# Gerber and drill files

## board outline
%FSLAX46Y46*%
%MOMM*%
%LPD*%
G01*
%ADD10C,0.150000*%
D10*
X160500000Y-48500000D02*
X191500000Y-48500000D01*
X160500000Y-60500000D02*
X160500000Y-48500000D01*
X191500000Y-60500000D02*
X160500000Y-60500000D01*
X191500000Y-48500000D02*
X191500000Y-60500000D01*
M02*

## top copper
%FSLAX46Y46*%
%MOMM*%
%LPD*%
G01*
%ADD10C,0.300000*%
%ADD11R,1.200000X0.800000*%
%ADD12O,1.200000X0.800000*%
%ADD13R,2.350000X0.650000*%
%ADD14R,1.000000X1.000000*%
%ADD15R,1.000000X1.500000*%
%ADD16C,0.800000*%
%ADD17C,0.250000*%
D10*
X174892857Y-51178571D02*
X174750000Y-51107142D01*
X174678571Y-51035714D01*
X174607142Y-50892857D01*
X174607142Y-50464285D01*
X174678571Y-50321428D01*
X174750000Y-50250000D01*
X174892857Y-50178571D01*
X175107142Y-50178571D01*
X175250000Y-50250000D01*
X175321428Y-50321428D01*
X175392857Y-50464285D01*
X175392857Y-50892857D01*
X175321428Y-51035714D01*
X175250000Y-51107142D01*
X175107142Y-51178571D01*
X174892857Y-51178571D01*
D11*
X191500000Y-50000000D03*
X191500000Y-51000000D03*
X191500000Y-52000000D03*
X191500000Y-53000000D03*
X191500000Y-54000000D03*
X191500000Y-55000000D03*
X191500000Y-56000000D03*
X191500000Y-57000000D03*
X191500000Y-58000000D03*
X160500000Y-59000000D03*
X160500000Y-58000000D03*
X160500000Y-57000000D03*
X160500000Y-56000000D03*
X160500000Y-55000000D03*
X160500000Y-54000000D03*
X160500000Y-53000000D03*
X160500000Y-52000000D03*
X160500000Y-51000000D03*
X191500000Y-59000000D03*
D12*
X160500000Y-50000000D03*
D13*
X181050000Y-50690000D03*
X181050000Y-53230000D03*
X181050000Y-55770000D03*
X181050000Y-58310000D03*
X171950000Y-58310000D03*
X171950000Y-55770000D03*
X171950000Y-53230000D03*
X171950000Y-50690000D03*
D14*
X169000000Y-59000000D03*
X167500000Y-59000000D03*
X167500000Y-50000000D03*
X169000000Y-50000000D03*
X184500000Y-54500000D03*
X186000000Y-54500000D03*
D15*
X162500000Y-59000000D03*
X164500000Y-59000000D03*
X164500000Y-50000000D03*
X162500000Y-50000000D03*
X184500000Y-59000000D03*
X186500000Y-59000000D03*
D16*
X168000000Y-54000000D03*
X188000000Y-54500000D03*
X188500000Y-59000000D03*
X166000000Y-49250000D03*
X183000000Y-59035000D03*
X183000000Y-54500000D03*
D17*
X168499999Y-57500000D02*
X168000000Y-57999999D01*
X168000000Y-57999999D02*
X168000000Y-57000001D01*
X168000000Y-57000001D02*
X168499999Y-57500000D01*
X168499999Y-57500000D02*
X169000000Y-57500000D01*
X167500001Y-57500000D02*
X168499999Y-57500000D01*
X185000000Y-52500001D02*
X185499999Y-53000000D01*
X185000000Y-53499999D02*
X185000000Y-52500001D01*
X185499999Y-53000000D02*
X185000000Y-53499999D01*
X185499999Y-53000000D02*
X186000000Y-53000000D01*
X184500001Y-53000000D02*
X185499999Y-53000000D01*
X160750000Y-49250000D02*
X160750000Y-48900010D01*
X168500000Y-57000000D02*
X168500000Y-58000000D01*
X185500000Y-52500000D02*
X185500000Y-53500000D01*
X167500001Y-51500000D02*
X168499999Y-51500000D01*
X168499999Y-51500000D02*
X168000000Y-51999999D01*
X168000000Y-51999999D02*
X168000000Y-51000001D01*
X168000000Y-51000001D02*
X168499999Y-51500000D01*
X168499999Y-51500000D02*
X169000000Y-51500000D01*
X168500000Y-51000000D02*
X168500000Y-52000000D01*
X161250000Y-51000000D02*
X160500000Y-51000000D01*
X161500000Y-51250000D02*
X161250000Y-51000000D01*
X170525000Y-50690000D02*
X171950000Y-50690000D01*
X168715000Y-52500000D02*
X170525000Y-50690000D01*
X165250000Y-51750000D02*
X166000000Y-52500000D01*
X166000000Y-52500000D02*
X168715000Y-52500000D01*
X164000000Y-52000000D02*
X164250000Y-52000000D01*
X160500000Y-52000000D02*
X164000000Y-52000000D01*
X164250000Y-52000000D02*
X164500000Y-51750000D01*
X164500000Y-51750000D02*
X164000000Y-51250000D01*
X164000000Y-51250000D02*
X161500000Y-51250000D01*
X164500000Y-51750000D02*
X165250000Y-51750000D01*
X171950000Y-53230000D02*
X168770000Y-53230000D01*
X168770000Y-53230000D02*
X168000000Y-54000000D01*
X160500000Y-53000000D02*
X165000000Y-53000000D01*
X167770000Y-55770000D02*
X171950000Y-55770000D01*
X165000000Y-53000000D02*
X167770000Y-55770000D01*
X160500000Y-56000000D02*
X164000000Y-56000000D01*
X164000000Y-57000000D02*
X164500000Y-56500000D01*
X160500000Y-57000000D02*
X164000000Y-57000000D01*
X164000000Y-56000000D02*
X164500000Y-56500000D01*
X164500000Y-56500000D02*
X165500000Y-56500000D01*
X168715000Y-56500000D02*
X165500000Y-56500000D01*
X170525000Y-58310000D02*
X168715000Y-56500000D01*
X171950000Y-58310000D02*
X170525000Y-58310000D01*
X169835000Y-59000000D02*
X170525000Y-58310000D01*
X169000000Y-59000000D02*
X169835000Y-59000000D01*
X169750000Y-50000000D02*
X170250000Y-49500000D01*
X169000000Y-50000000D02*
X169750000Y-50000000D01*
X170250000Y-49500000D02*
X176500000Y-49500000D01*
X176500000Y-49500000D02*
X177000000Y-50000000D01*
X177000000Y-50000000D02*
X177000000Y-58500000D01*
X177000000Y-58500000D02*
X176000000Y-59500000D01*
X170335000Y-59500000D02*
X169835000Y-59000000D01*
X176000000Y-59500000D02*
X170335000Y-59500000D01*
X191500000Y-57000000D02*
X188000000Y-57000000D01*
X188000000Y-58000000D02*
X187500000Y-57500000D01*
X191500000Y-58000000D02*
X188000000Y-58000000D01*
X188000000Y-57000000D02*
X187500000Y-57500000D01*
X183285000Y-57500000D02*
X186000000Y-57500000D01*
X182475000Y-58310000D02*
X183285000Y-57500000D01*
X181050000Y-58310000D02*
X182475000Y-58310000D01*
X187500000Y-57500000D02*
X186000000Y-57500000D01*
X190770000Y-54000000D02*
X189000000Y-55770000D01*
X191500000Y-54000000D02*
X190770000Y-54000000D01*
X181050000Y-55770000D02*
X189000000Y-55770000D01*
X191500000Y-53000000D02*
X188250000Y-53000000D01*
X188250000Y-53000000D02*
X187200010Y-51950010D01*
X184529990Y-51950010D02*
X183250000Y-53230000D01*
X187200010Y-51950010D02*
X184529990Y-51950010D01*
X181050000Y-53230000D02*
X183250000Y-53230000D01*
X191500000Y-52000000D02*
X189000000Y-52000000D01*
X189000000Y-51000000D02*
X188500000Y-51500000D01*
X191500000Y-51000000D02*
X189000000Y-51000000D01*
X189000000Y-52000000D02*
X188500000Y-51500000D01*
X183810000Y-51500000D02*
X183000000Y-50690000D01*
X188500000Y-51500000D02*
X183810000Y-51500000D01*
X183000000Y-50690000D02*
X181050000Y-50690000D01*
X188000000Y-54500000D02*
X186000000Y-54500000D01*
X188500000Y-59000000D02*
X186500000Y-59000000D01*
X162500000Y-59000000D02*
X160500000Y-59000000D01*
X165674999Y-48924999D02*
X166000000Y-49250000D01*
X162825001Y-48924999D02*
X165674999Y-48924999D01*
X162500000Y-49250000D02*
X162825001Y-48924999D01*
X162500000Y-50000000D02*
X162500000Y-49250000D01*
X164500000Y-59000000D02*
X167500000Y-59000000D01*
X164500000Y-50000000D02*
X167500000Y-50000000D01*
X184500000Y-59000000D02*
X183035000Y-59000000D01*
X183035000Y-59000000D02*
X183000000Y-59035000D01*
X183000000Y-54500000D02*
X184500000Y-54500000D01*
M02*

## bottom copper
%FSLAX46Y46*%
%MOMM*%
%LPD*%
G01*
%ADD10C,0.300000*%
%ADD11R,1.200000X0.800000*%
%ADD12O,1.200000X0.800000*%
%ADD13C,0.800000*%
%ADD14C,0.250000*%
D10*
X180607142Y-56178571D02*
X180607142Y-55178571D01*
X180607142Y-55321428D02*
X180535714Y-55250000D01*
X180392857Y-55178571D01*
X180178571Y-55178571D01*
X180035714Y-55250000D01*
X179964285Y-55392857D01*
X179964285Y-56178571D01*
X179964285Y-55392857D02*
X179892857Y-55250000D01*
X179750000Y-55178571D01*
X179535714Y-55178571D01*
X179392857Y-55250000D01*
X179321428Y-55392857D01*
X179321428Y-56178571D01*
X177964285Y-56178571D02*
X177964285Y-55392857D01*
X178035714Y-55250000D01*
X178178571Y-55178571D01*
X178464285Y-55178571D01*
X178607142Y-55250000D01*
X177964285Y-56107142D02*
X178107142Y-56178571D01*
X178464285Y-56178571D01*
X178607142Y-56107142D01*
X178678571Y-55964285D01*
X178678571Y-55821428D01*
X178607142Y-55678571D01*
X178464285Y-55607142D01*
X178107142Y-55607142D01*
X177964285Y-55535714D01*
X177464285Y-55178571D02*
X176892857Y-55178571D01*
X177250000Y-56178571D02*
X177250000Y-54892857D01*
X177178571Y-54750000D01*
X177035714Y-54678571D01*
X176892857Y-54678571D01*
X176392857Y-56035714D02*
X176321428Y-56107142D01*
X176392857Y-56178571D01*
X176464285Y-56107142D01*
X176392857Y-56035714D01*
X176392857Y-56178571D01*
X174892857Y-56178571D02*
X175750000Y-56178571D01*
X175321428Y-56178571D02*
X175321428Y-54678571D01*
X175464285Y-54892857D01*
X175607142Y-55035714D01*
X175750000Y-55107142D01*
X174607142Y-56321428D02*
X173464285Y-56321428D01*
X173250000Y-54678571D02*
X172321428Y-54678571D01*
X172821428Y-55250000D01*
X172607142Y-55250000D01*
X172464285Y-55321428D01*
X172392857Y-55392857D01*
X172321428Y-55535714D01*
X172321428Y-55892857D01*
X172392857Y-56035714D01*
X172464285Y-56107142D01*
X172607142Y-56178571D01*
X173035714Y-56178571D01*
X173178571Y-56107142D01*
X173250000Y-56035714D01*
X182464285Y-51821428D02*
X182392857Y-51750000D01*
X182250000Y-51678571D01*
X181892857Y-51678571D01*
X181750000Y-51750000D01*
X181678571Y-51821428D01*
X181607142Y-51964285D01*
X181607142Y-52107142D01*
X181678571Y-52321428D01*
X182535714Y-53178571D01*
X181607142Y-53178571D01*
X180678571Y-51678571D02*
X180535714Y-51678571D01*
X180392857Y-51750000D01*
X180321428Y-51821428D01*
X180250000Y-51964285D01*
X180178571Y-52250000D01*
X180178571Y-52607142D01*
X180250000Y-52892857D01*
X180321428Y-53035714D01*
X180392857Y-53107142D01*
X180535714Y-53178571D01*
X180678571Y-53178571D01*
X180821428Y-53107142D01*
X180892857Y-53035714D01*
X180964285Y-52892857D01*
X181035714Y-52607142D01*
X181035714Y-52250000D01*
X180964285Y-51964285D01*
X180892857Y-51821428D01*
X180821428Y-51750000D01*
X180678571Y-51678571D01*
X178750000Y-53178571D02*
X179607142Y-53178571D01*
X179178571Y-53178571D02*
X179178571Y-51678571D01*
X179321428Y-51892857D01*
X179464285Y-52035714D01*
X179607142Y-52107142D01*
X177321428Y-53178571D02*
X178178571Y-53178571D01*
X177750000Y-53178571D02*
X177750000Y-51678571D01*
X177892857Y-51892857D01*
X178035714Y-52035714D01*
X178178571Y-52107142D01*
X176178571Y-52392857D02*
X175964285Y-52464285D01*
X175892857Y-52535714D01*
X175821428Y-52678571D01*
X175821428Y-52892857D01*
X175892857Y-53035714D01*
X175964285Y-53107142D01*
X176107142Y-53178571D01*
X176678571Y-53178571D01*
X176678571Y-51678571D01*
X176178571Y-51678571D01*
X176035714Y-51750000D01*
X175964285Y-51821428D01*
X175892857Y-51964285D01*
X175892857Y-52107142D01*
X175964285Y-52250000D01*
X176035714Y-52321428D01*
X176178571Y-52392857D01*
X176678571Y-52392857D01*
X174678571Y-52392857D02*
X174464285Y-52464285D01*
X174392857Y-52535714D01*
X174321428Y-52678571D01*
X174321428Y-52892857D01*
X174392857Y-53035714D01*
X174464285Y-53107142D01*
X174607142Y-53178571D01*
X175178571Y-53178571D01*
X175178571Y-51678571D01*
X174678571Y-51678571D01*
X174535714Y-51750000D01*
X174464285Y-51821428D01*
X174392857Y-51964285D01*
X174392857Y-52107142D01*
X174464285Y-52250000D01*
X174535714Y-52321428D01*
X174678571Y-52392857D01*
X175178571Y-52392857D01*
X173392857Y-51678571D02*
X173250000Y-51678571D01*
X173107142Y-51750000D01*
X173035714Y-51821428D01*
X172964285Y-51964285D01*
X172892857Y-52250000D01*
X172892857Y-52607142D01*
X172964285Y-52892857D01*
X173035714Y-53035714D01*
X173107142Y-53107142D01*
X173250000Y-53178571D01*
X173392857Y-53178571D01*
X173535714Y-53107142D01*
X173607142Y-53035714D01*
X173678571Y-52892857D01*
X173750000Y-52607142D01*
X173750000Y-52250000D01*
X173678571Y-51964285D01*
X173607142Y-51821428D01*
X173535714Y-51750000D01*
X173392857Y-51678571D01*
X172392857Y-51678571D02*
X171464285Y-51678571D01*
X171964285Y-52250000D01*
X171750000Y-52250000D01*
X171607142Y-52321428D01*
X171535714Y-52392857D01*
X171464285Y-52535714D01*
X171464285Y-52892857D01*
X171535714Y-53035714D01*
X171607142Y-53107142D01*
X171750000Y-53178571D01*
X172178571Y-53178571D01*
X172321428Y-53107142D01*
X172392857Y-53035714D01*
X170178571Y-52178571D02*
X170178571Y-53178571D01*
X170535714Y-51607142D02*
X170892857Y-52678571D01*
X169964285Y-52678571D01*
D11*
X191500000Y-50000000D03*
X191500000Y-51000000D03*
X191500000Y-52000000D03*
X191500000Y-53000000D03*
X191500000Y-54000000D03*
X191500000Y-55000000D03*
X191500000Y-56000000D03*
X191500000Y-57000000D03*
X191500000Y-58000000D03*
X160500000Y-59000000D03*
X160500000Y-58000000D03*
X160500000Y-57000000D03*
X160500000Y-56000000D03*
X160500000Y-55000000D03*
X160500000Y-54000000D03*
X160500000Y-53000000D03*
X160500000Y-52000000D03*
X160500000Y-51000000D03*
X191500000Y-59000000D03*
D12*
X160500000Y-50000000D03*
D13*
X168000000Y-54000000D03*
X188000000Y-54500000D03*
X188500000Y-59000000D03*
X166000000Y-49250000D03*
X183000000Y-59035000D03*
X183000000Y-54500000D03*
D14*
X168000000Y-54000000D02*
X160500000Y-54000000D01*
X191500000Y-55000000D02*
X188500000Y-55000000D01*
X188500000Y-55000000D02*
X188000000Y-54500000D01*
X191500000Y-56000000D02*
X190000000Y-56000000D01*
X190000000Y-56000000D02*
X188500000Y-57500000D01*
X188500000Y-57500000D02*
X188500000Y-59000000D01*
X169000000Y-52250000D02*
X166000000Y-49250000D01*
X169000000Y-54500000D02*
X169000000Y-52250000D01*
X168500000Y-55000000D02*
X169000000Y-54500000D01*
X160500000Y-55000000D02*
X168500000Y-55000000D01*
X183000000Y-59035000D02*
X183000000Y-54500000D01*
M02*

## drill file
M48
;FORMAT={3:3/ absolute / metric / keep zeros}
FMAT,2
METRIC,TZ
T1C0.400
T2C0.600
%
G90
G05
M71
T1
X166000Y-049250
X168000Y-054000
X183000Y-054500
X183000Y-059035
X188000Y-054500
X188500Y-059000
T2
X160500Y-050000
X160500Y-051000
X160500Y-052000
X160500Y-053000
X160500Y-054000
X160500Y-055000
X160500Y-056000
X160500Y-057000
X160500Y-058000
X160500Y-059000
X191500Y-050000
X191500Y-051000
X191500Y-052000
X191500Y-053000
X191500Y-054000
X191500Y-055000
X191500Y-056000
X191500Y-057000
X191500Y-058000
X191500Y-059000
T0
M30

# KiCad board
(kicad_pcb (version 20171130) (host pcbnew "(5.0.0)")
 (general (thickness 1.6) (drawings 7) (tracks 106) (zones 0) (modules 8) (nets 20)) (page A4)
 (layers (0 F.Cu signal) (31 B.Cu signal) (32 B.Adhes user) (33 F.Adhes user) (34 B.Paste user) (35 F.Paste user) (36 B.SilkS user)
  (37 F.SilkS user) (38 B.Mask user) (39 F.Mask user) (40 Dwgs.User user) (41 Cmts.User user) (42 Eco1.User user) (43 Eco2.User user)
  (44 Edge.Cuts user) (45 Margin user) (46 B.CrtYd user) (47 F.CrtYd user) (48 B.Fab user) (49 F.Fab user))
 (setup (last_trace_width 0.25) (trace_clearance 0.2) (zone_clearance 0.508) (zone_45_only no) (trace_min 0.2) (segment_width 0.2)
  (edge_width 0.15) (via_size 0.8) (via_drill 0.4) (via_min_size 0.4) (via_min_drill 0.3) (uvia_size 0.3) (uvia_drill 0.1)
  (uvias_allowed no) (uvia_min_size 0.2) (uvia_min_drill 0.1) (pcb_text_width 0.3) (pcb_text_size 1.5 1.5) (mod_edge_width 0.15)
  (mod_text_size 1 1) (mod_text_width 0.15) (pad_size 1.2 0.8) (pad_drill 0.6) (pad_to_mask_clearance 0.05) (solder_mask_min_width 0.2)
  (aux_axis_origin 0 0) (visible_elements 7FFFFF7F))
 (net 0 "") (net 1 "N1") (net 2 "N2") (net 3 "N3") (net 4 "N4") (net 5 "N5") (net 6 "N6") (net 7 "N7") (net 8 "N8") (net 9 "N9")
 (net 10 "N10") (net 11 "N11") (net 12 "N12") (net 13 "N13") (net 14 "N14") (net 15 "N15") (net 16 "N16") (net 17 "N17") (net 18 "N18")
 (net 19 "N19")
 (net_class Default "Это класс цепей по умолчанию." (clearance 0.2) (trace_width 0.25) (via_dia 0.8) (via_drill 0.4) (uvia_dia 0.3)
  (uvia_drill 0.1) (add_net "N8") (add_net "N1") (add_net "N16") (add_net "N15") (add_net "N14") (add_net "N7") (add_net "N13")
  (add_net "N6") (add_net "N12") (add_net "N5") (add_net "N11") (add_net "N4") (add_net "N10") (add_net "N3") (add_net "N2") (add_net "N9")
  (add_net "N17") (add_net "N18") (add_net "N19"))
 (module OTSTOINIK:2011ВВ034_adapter (layer F.Cu) (at 176 54.5)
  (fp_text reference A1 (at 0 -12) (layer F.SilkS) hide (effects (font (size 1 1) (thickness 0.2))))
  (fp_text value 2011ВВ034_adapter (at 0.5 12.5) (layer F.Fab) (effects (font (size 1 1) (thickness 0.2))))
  (pad 10B thru_hole rect (at 15.5 -4.5) (size 1.2 0.8) (drill 0.6) (layers *.Cu *.Mask) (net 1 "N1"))
  (pad 9B thru_hole rect (at 15.5 -3.5) (size 1.2 0.8) (drill 0.6) (layers *.Cu *.Mask) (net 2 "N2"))
  (pad 8B thru_hole rect (at 15.5 -2.5) (size 1.2 0.8) (drill 0.6) (layers *.Cu *.Mask) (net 2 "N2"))
  (pad 7B thru_hole rect (at 15.5 -1.5) (size 1.2 0.8) (drill 0.6) (layers *.Cu *.Mask) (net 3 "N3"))
  (pad 6B thru_hole rect (at 15.5 -0.5) (size 1.2 0.8) (drill 0.6) (layers *.Cu *.Mask) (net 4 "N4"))
  (pad 5B thru_hole rect (at 15.5 0.5) (size 1.2 0.8) (drill 0.6) (layers *.Cu *.Mask) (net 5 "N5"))
  (pad 4B thru_hole rect (at 15.5 1.5) (size 1.2 0.8) (drill 0.6) (layers *.Cu *.Mask) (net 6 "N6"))
  (pad 3B thru_hole rect (at 15.5 2.5) (size 1.2 0.8) (drill 0.6) (layers *.Cu *.Mask) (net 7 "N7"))
  (pad 2B thru_hole rect (at 15.5 3.5) (size 1.2 0.8) (drill 0.6) (layers *.Cu *.Mask) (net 7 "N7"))
  (pad 10A thru_hole rect (at -15.5 4.5) (size 1.2 0.8) (drill 0.6) (layers *.Cu *.Mask) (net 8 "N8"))
  (pad 9A thru_hole rect (at -15.5 3.5) (size 1.2 0.8) (drill 0.6) (layers *.Cu *.Mask) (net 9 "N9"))
  (pad 8A thru_hole rect (at -15.5 2.5) (size 1.2 0.8) (drill 0.6) (layers *.Cu *.Mask) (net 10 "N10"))
  (pad 7A thru_hole rect (at -15.5 1.5) (size 1.2 0.8) (drill 0.6) (layers *.Cu *.Mask) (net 10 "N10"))
  (pad 6A thru_hole rect (at -15.5 0.5) (size 1.2 0.8) (drill 0.6) (layers *.Cu *.Mask) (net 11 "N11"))
  (pad 5A thru_hole rect (at -15.5 -0.5) (size 1.2 0.8) (drill 0.6) (layers *.Cu *.Mask) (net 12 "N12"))
  (pad 4A thru_hole rect (at -15.5 -1.5) (size 1.2 0.8) (drill 0.6) (layers *.Cu *.Mask) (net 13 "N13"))
  (pad 3A thru_hole rect (at -15.5 -2.5) (size 1.2 0.8) (drill 0.6) (layers *.Cu *.Mask) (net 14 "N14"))
  (pad 2A thru_hole rect (at -15.5 -3.5) (size 1.2 0.8) (drill 0.6) (layers *.Cu *.Mask) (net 14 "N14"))
  (pad 1B thru_hole rect (at 15.5 4.5) (size 1.2 0.8) (drill 0.6) (layers *.Cu *.Mask) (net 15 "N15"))
  (pad 1A thru_hole oval (at -15.5 -4.5) (size 1.2 0.8) (drill 0.6) (layers *.Cu *.Mask) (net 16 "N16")))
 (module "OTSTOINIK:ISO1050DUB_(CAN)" (layer F.Cu) (at 176.5 54.5)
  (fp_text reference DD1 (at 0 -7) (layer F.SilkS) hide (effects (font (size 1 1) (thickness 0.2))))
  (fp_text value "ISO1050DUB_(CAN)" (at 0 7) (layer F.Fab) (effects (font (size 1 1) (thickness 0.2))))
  (pad 8 smd rect (at 4.55 -3.81) (size 2.35 0.65) (layers F.Cu F.Paste F.Mask) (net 2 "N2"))
  (pad 7 smd rect (at 4.55 -1.27) (size 2.35 0.65) (layers F.Cu F.Paste F.Mask) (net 3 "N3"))
  (pad 6 smd rect (at 4.55 1.27) (size 2.35 0.65) (layers F.Cu F.Paste F.Mask) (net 4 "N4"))
  (pad 5 smd rect (at 4.55 3.81) (size 2.35 0.65) (layers F.Cu F.Paste F.Mask) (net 7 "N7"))
  (pad 4 smd rect (at -4.55 3.81) (size 2.35 0.65) (layers F.Cu F.Paste F.Mask) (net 10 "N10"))
  (pad 3 smd rect (at -4.55 1.27) (size 2.35 0.65) (layers F.Cu F.Paste F.Mask) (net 13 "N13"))
  (pad 2 smd rect (at -4.55 -1.27) (size 2.35 0.65) (layers F.Cu F.Paste F.Mask) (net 12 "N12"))
  (pad 1 smd rect (at -4.55 -3.81) (size 2.35 0.65) (layers F.Cu F.Paste F.Mask) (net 14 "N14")))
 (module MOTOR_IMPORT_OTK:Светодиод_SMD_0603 (layer F.Cu) (at 167.5 59)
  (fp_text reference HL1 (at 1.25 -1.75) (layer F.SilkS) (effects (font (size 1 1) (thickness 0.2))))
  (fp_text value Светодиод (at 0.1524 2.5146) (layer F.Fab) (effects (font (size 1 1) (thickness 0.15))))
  (pad 2 smd rect (at 1.5 0) (size 1 1) (layers F.Cu F.Paste F.Mask) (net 10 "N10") (clearance 0.2))
  (pad 1 smd rect (at 0 0) (size 1 1) (layers F.Cu F.Paste F.Mask) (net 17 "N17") (clearance 0.2)))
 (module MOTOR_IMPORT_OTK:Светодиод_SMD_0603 (layer F.Cu) (at 167.5 50)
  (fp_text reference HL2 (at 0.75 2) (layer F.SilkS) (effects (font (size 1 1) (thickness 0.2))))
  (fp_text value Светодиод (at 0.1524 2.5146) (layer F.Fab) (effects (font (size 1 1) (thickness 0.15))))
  (pad 1 smd rect (at 0 0) (size 1 1) (layers F.Cu F.Paste F.Mask) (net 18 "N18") (clearance 0.2))
  (pad 2 smd rect (at 1.5 0) (size 1 1) (layers F.Cu F.Paste F.Mask) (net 10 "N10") (clearance 0.2)))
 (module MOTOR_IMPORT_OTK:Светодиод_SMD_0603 (layer F.Cu) (at 184.5 54.5)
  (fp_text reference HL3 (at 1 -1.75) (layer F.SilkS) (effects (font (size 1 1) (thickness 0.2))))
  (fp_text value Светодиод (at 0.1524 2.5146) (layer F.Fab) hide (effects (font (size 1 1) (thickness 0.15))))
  (pad 1 smd rect (at 0 0) (size 1 1) (layers F.Cu F.Paste F.Mask) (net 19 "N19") (clearance 0.2))
  (pad 2 smd rect (at 1.5 0) (size 1 1) (layers F.Cu F.Paste F.Mask) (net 5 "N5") (clearance 0.2)))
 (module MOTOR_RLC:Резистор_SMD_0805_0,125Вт (layer F.Cu) (at 164.5 59 180)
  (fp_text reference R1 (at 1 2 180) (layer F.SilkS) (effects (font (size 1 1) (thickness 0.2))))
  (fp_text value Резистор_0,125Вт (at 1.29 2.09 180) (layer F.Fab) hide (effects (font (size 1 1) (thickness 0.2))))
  (pad 2 smd rect (at 2 0 180) (size 1 1.5) (layers F.Cu F.Paste F.Mask) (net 8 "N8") (clearance 0.2))
  (pad 1 smd rect (at 0 0 180) (size 1 1.5) (layers F.Cu F.Paste F.Mask) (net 17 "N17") (clearance 0.2)))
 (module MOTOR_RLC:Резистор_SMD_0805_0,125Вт (layer F.Cu) (at 164.5 50 180)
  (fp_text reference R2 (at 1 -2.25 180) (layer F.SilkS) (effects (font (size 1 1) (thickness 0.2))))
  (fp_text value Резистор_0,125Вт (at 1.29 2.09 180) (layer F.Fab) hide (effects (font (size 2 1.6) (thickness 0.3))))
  (pad 1 smd rect (at 0 0 180) (size 1 1.5) (layers F.Cu F.Paste F.Mask) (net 18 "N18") (clearance 0.2))
  (pad 2 smd rect (at 2 0 180) (size 1 1.5) (layers F.Cu F.Paste F.Mask) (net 11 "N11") (clearance 0.2)))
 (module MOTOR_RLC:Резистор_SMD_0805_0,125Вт (layer F.Cu) (at 186.5 59 180)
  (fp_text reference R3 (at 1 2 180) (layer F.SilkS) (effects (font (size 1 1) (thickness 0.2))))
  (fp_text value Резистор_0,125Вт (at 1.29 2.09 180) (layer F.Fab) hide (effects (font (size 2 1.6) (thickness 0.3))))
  (pad 2 smd rect (at 2 0 180) (size 1 1.5) (layers F.Cu F.Paste F.Mask) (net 19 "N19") (clearance 0.2))
  (pad 1 smd rect (at 0 0 180) (size 1 1.5) (layers F.Cu F.Paste F.Mask) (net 6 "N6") (clearance 0.2)))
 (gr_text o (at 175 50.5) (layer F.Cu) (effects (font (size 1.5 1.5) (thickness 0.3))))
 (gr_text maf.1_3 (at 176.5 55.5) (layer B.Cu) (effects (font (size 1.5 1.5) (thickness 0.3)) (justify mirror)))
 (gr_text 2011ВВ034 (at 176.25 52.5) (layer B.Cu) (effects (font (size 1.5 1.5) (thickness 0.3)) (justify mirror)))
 (gr_line (start 160.5 48.5) (end 191.5 48.5) (layer Edge.Cuts) (width 0.15))
 (gr_line (start 160.5 60.5) (end 160.5 48.5) (layer Edge.Cuts) (width 0.15))
 (gr_line (start 191.5 60.5) (end 160.5 60.5) (layer Edge.Cuts) (width 0.15))
 (gr_line (start 191.5 48.5) (end 191.5 60.5) (layer Edge.Cuts) (width 0.15))
 (segment (start 168.499999 57.5) (end 168 57.999999) (width 0.25) (layer F.Cu) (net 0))
 (segment (start 168 57.999999) (end 168 57.000001) (width 0.25) (layer F.Cu) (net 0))
 (segment (start 168 57.000001) (end 168.499999 57.5) (width 0.25) (layer F.Cu) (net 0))
 (segment (start 168.499999 57.5) (end 169 57.5) (width 0.25) (layer F.Cu) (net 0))
 (segment (start 167.500001 57.5) (end 168.499999 57.5) (width 0.25) (layer F.Cu) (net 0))
 (segment (start 185 52.500001) (end 185.499999 53) (width 0.25) (layer F.Cu) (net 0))
 (segment (start 185 53.499999) (end 185 52.500001) (width 0.25) (layer F.Cu) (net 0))
 (segment (start 185.499999 53) (end 185 53.499999) (width 0.25) (layer F.Cu) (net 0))
 (segment (start 185.499999 53) (end 186 53) (width 0.25) (layer F.Cu) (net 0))
 (segment (start 184.500001 53) (end 185.499999 53) (width 0.25) (layer F.Cu) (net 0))
 (segment (start 160.75 49.25) (end 160.75 48.90001) (width 0.25) (layer F.Cu) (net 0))
 (segment (start 168.5 57) (end 168.5 58) (width 0.25) (layer F.Cu) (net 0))
 (segment (start 185.5 52.5) (end 185.5 53.5) (width 0.25) (layer F.Cu) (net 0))
 (segment (start 167.500001 51.5) (end 168.499999 51.5) (width 0.25) (layer F.Cu) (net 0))
 (segment (start 168.499999 51.5) (end 168 51.999999) (width 0.25) (layer F.Cu) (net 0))
 (segment (start 168 51.999999) (end 168 51.000001) (width 0.25) (layer F.Cu) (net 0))
 (segment (start 168 51.000001) (end 168.499999 51.5) (width 0.25) (layer F.Cu) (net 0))
 (segment (start 168.499999 51.5) (end 169 51.5) (width 0.25) (layer F.Cu) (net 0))
 (segment (start 168.5 51) (end 168.5 52) (width 0.25) (layer F.Cu) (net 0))
 (segment (start 161.25 51) (end 160.5 51) (width 0.25) (layer F.Cu) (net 14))
 (segment (start 161.5 51.25) (end 161.25 51) (width 0.25) (layer F.Cu) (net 14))
 (segment (start 170.525 50.69) (end 171.95 50.69) (width 0.25) (layer F.Cu) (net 14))
 (segment (start 168.715 52.5) (end 170.525 50.69) (width 0.25) (layer F.Cu) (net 14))
 (segment (start 165.25 51.75) (end 166 52.5) (width 0.25) (layer F.Cu) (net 14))
 (segment (start 166 52.5) (end 168.715 52.5) (width 0.25) (layer F.Cu) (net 14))
 (segment (start 164 52) (end 164.25 52) (width 0.25) (layer F.Cu) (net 14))
 (segment (start 160.5 52) (end 164 52) (width 0.25) (layer F.Cu) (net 14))
 (segment (start 164.25 52) (end 164.5 51.75) (width 0.25) (layer F.Cu) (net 14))
 (segment (start 164.5 51.75) (end 164 51.25) (width 0.25) (layer F.Cu) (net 14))
 (segment (start 164 51.25) (end 161.5 51.25) (width 0.25) (layer F.Cu) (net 14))
 (segment (start 164.5 51.75) (end 165.25 51.75) (width 0.25) (layer F.Cu) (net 14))
 (via (at 168 54) (size 0.8) (drill 0.4) (layers F.Cu B.Cu) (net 12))
 (segment (start 171.95 53.23) (end 168.77 53.23) (width 0.25) (layer F.Cu) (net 12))
 (segment (start 168.77 53.23) (end 168 54) (width 0.25) (layer F.Cu) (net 12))
 (segment (start 168 54) (end 160.5 54) (width 0.25) (layer B.Cu) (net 12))
 (segment (start 160.5 53) (end 165 53) (width 0.25) (layer F.Cu) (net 13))
 (segment (start 167.77 55.77) (end 171.95 55.77) (width 0.25) (layer F.Cu) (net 13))
 (segment (start 165 53) (end 167.77 55.77) (width 0.25) (layer F.Cu) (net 13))
 (segment (start 160.5 56) (end 164 56) (width 0.25) (layer F.Cu) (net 10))
 (segment (start 164 57) (end 164.5 56.5) (width 0.25) (layer F.Cu) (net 10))
 (segment (start 160.5 57) (end 164 57) (width 0.25) (layer F.Cu) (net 10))
 (segment (start 164 56) (end 164.5 56.5) (width 0.25) (layer F.Cu) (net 10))
 (segment (start 164.5 56.5) (end 165.5 56.5) (width 0.25) (layer F.Cu) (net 10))
 (segment (start 168.715 56.5) (end 165.5 56.5) (width 0.25) (layer F.Cu) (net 10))
 (segment (start 170.525 58.31) (end 168.715 56.5) (width 0.25) (layer F.Cu) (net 10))
 (segment (start 171.95 58.31) (end 170.525 58.31) (width 0.25) (layer F.Cu) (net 10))
 (segment (start 169.835 59) (end 170.525 58.31) (width 0.25) (layer F.Cu) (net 10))
 (segment (start 169 59) (end 169.835 59) (width 0.25) (layer F.Cu) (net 10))
 (segment (start 169.75 50) (end 170.25 49.5) (width 0.25) (layer F.Cu) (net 10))
 (segment (start 169 50) (end 169.75 50) (width 0.25) (layer F.Cu) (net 10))
 (segment (start 170.25 49.5) (end 176.5 49.5) (width 0.25) (layer F.Cu) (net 10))
 (segment (start 176.5 49.5) (end 177 50) (width 0.25) (layer F.Cu) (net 10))
 (segment (start 177 50) (end 177 58.5) (width 0.25) (layer F.Cu) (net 10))
 (segment (start 177 58.5) (end 176 59.5) (width 0.25) (layer F.Cu) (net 10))
 (segment (start 170.335 59.5) (end 169.835 59) (width 0.25) (layer F.Cu) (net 10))
 (segment (start 176 59.5) (end 170.335 59.5) (width 0.25) (layer F.Cu) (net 10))
 (segment (start 191.5 57) (end 188 57) (width 0.25) (layer F.Cu) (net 7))
 (segment (start 188 58) (end 187.5 57.5) (width 0.25) (layer F.Cu) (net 7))
 (segment (start 191.5 58) (end 188 58) (width 0.25) (layer F.Cu) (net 7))
 (segment (start 188 57) (end 187.5 57.5) (width 0.25) (layer F.Cu) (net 7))
 (segment (start 183.285 57.5) (end 186 57.5) (width 0.25) (layer F.Cu) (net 7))
 (segment (start 182.475 58.31) (end 183.285 57.5) (width 0.25) (layer F.Cu) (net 7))
 (segment (start 181.05 58.31) (end 182.475 58.31) (width 0.25) (layer F.Cu) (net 7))
 (segment (start 187.5 57.5) (end 186 57.5) (width 0.25) (layer F.Cu) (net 7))
 (segment (start 190.77 54) (end 189 55.77) (width 0.25) (layer F.Cu) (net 4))
 (segment (start 191.5 54) (end 190.77 54) (width 0.25) (layer F.Cu) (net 4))
 (segment (start 181.05 55.77) (end 189 55.77) (width 0.25) (layer F.Cu) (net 4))
 (segment (start 191.5 53) (end 188.25 53) (width 0.25) (layer F.Cu) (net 3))
 (segment (start 188.25 53) (end 187.20001 51.95001) (width 0.25) (layer F.Cu) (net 3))
 (segment (start 184.52999 51.95001) (end 183.25 53.23) (width 0.25) (layer F.Cu) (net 3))
 (segment (start 187.20001 51.95001) (end 184.52999 51.95001) (width 0.25) (layer F.Cu) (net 3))
 (segment (start 181.05 53.23) (end 183.25 53.23) (width 0.25) (layer F.Cu) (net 3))
 (segment (start 191.5 52) (end 189 52) (width 0.25) (layer F.Cu) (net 2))
 (segment (start 189 51) (end 188.5 51.5) (width 0.25) (layer F.Cu) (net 2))
 (segment (start 191.5 51) (end 189 51) (width 0.25) (layer F.Cu) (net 2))
 (segment (start 189 52) (end 188.5 51.5) (width 0.25) (layer F.Cu) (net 2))
 (segment (start 183.81 51.5) (end 183 50.69) (width 0.25) (layer F.Cu) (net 2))
 (segment (start 188.5 51.5) (end 183.81 51.5) (width 0.25) (layer F.Cu) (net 2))
 (segment (start 183 50.69) (end 181.05 50.69) (width 0.25) (layer F.Cu) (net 2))
 (via (at 188 54.5) (size 0.8) (drill 0.4) (layers F.Cu B.Cu) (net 5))
 (segment (start 191.5 55) (end 188.5 55) (width 0.25) (layer B.Cu) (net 5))
 (segment (start 188.5 55) (end 188 54.5) (width 0.25) (layer B.Cu) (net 5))
 (segment (start 188 54.5) (end 186 54.5) (width 0.25) (layer F.Cu) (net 5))
 (segment (start 191.5 56) (end 190 56) (width 0.25) (layer B.Cu) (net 6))
 (via (at 188.5 59) (size 0.8) (drill 0.4) (layers F.Cu B.Cu) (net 6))
 (segment (start 190 56) (end 188.5 57.5) (width 0.25) (layer B.Cu) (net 6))
 (segment (start 188.5 57.5) (end 188.5 59) (width 0.25) (layer B.Cu) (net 6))
 (segment (start 188.5 59) (end 186.5 59) (width 0.25) (layer F.Cu) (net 6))
 (segment (start 162.5 59) (end 160.5 59) (width 0.25) (layer F.Cu) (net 8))
 (via (at 166 49.25) (size 0.8) (drill 0.4) (layers F.Cu B.Cu) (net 11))
 (segment (start 165.674999 48.924999) (end 166 49.25) (width 0.25) (layer F.Cu) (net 11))
 (segment (start 162.825001 48.924999) (end 165.674999 48.924999) (width 0.25) (layer F.Cu) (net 11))
 (segment (start 162.5 49.25) (end 162.825001 48.924999) (width 0.25) (layer F.Cu) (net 11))
 (segment (start 162.5 50) (end 162.5 49.25) (width 0.25) (layer F.Cu) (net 11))
 (segment (start 169 52.25) (end 166 49.25) (width 0.25) (layer B.Cu) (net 11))
 (segment (start 169 54.5) (end 169 52.25) (width 0.25) (layer B.Cu) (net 11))
 (segment (start 168.5 55) (end 169 54.5) (width 0.25) (layer B.Cu) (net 11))
 (segment (start 160.5 55) (end 168.5 55) (width 0.25) (layer B.Cu) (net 11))
 (segment (start 164.5 59) (end 167.5 59) (width 0.25) (layer F.Cu) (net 17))
 (segment (start 164.5 50) (end 167.5 50) (width 0.25) (layer F.Cu) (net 18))
 (via (at 183 59.035) (size 0.8) (drill 0.4) (layers F.Cu B.Cu) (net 19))
 (segment (start 184.5 59) (end 183.035 59) (width 0.25) (layer F.Cu) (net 19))
 (segment (start 183.035 59) (end 183 59.035) (width 0.25) (layer F.Cu) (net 19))
 (via (at 183 54.5) (size 0.8) (drill 0.4) (layers F.Cu B.Cu) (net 19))
 (segment (start 183 59.035) (end 183 54.5) (width 0.25) (layer B.Cu) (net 19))
 (segment (start 183 54.5) (end 184.5 54.5) (width 0.25) (layer F.Cu) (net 19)))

